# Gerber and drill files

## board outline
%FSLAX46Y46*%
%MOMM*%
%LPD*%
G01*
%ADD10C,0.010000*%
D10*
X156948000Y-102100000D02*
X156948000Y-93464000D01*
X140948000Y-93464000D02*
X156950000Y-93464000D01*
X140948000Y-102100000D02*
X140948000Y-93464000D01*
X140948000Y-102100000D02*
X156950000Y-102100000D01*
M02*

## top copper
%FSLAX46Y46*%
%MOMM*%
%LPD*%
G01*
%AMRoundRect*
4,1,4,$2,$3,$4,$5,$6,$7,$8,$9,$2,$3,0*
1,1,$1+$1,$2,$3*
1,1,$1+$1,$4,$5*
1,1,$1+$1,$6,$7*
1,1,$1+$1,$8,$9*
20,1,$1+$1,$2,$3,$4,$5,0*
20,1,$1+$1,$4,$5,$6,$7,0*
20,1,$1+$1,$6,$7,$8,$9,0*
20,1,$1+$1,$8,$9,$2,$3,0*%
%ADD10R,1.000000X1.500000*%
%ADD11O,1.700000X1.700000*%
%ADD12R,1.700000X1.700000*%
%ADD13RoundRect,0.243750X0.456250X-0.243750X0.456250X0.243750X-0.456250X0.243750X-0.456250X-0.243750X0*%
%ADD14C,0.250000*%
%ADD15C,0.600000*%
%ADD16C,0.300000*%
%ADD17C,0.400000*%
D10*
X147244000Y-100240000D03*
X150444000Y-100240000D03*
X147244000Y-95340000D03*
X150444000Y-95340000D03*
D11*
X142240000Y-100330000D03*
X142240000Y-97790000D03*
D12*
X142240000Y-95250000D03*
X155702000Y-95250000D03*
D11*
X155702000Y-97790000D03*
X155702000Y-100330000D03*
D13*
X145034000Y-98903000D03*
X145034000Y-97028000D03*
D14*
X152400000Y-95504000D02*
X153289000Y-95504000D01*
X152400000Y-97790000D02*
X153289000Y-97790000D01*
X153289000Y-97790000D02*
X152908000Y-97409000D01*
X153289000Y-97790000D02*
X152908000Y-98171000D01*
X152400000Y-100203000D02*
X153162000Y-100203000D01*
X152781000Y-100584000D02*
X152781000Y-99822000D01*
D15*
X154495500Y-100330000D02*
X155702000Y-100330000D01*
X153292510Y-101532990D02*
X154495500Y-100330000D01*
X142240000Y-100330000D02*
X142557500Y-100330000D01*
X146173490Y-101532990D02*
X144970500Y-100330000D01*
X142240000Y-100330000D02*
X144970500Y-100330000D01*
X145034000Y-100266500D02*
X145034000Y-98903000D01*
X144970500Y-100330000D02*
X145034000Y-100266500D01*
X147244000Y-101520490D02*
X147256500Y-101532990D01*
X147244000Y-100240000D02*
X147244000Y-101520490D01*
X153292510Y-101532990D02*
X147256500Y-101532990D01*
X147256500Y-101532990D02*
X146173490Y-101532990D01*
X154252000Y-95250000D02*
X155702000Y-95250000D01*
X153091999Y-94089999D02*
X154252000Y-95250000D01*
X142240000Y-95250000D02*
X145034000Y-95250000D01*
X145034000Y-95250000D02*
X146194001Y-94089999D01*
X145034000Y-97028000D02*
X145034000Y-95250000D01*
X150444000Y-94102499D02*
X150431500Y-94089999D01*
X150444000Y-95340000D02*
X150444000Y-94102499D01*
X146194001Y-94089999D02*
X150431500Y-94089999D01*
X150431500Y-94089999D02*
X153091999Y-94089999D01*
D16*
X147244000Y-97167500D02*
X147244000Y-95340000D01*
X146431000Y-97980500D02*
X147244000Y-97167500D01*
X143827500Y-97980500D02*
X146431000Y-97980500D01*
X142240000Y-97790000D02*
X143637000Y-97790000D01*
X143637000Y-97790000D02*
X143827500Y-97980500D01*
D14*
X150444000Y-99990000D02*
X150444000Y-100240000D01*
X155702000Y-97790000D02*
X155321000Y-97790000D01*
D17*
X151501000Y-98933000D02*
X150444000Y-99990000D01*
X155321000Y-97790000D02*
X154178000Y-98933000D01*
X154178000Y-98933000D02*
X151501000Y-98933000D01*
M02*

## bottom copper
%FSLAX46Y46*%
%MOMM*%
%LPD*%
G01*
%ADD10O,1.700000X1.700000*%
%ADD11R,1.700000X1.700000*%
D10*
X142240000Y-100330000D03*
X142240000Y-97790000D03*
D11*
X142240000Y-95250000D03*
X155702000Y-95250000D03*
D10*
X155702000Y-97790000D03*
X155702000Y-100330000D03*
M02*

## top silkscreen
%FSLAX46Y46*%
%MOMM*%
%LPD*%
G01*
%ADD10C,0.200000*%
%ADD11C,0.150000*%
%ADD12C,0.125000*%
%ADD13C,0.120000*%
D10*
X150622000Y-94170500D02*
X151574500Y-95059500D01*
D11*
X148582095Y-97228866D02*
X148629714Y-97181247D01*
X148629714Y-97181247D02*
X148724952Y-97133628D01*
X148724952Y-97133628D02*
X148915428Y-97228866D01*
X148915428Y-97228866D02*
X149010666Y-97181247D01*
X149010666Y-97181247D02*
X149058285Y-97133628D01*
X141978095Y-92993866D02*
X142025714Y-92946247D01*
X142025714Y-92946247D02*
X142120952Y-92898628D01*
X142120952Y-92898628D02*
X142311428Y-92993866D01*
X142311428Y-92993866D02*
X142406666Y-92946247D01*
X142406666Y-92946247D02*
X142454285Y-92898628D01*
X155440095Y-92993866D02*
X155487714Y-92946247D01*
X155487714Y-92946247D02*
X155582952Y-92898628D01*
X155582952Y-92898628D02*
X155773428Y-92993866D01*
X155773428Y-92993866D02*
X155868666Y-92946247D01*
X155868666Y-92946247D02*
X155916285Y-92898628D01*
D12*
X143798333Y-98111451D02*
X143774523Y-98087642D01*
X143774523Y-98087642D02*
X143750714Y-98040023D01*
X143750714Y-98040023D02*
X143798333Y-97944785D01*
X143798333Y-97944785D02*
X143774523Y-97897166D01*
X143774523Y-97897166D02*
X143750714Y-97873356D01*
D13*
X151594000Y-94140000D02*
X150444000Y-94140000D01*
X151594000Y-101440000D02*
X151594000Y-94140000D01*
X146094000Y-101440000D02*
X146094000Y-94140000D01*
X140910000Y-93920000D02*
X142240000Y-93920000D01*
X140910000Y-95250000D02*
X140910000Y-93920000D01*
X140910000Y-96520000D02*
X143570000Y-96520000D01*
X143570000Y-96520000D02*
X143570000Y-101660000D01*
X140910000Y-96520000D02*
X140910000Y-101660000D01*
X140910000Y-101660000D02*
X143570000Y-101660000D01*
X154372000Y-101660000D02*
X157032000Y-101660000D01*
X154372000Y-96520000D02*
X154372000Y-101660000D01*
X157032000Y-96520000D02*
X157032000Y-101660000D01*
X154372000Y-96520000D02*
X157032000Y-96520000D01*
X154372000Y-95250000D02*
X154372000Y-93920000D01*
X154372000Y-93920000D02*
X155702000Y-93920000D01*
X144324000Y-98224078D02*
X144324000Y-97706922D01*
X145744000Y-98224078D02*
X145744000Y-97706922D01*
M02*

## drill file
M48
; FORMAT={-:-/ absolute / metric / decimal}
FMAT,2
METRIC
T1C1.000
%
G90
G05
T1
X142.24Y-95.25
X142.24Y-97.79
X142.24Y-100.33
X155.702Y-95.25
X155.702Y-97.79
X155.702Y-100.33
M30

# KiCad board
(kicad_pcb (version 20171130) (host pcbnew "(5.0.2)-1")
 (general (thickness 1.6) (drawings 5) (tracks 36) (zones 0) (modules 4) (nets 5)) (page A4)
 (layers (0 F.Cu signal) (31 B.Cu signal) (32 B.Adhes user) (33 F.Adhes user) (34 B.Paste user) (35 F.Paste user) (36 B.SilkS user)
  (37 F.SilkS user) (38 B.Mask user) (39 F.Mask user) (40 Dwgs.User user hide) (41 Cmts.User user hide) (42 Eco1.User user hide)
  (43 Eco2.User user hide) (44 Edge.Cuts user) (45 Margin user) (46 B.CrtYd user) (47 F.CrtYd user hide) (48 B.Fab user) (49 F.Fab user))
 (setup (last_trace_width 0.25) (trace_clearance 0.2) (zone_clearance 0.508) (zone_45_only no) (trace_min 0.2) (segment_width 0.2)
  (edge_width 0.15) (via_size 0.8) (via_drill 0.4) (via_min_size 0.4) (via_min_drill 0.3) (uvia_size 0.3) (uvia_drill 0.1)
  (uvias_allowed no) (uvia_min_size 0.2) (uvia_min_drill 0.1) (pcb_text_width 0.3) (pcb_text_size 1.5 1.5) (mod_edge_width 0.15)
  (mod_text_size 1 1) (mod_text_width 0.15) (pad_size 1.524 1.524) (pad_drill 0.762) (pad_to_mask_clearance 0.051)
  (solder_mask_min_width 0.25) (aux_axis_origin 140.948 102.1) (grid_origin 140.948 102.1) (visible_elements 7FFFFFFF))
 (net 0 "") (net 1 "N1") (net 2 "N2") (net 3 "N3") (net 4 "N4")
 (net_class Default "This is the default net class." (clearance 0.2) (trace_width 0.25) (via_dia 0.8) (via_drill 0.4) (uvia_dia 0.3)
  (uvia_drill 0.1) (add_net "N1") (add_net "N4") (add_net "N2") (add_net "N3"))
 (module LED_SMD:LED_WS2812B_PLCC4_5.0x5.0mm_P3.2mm (layer F.Cu) (at 148.844 97.79 90)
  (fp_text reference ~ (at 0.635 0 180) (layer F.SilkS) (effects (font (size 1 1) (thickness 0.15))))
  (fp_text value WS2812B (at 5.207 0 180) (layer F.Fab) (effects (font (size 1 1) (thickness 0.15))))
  (fp_line (start 3.65 2.75) (end 3.65 1.6) (layer F.SilkS) (width 0.12))
  (fp_line (start -3.65 2.75) (end 3.65 2.75) (layer F.SilkS) (width 0.12))
  (fp_line (start -3.65 -2.75) (end 3.65 -2.75) (layer F.SilkS) (width 0.12))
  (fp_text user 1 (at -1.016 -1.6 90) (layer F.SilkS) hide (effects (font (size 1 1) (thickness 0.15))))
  (pad 1 smd rect (at -2.45 -1.6 90) (size 1.5 1) (layers F.Cu F.Paste F.Mask) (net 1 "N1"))
  (pad 2 smd rect (at -2.45 1.6 90) (size 1.5 1) (layers F.Cu F.Paste F.Mask) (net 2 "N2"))
  (pad 4 smd rect (at 2.45 -1.6 90) (size 1.5 1) (layers F.Cu F.Paste F.Mask) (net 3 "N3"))
  (pad 3 smd rect (at 2.45 1.6 90) (size 1.5 1) (layers F.Cu F.Paste F.Mask) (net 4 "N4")))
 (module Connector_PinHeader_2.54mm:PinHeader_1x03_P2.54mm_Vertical (layer F.Cu) (at 142.24 95.25)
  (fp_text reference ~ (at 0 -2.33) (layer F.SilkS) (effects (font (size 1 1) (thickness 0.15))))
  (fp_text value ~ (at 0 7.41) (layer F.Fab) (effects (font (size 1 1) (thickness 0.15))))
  (fp_line (start -1.33 -1.33) (end 0 -1.33) (layer F.SilkS) (width 0.12))
  (fp_line (start -1.33 0) (end -1.33 -1.33) (layer F.SilkS) (width 0.12))
  (fp_line (start -1.33 1.27) (end 1.33 1.27) (layer F.SilkS) (width 0.12))
  (fp_line (start 1.33 1.27) (end 1.33 6.41) (layer F.SilkS) (width 0.12))
  (fp_line (start -1.33 1.27) (end -1.33 6.41) (layer F.SilkS) (width 0.12))
  (fp_line (start -1.33 6.41) (end 1.33 6.41) (layer F.SilkS) (width 0.12))
  (pad 3 thru_hole oval (at 0 5.08) (size 1.7 1.7) (drill 1) (layers *.Cu *.Mask) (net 1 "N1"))
  (pad 2 thru_hole oval (at 0 2.54) (size 1.7 1.7) (drill 1) (layers *.Cu *.Mask) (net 3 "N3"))
  (pad 1 thru_hole rect (at 0 0) (size 1.7 1.7) (drill 1) (layers *.Cu *.Mask) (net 4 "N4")))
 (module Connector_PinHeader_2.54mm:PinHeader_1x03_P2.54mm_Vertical (layer F.Cu) (at 155.702 95.25)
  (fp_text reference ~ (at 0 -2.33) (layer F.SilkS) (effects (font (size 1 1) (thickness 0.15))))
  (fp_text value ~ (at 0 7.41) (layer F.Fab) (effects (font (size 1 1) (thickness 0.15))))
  (fp_line (start -1.33 6.41) (end 1.33 6.41) (layer F.SilkS) (width 0.12))
  (fp_line (start -1.33 1.27) (end -1.33 6.41) (layer F.SilkS) (width 0.12))
  (fp_line (start 1.33 1.27) (end 1.33 6.41) (layer F.SilkS) (width 0.12))
  (fp_line (start -1.33 1.27) (end 1.33 1.27) (layer F.SilkS) (width 0.12))
  (fp_line (start -1.33 0) (end -1.33 -1.33) (layer F.SilkS) (width 0.12))
  (fp_line (start -1.33 -1.33) (end 0 -1.33) (layer F.SilkS) (width 0.12))
  (pad 1 thru_hole rect (at 0 0) (size 1.7 1.7) (drill 1) (layers *.Cu *.Mask) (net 4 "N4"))
  (pad 2 thru_hole oval (at 0 2.54) (size 1.7 1.7) (drill 1) (layers *.Cu *.Mask) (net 2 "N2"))
  (pad 3 thru_hole oval (at 0 5.08) (size 1.7 1.7) (drill 1) (layers *.Cu *.Mask) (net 1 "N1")))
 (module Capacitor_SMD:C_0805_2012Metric (layer F.Cu) (at 145.034 97.9655 90)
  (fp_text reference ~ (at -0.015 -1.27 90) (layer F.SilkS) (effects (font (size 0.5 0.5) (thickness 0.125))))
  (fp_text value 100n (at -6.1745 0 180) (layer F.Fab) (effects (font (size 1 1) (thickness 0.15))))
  (fp_line (start -0.258578 -0.71) (end 0.258578 -0.71) (layer F.SilkS) (width 0.12))
  (fp_line (start -0.258578 0.71) (end 0.258578 0.71) (layer F.SilkS) (width 0.12))
  (pad 1 smd roundrect (at -0.9375 0 90) (size 0.975 1.4) (layers F.Cu F.Paste F.Mask) (roundrect_rratio 0.25) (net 1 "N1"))
  (pad 2 smd roundrect (at 0.9375 0 90) (size 0.975 1.4) (layers F.Cu F.Paste F.Mask) (roundrect_rratio 0.25) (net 4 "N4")))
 (gr_line (start 156.948 102.1) (end 156.948 93.464) (layer Edge.Cuts) (width 0.01))
 (gr_line (start 150.622 94.1705) (end 151.5745 95.0595) (layer F.SilkS) (width 0.2))
 (gr_line (start 140.948 93.464) (end 156.95 93.464) (layer Edge.Cuts) (width 0.01))
 (gr_line (start 140.948 102.1) (end 140.948 93.464) (layer Edge.Cuts) (width 0.01))
 (gr_line (start 140.948 102.1) (end 156.95 102.1) (layer Edge.Cuts) (width 0.01))
 (segment (start 152.4 95.504) (end 153.289 95.504) (width 0.25) (layer F.Cu) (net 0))
 (segment (start 152.4 97.79) (end 153.289 97.79) (width 0.25) (layer F.Cu) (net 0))
 (segment (start 153.289 97.79) (end 152.908 97.409) (width 0.25) (layer F.Cu) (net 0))
 (segment (start 153.289 97.79) (end 152.908 98.171) (width 0.25) (layer F.Cu) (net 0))
 (segment (start 152.4 100.203) (end 153.162 100.203) (width 0.25) (layer F.Cu) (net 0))
 (segment (start 152.781 100.584) (end 152.781 99.822) (width 0.25) (layer F.Cu) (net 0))
 (segment (start 154.4955 100.33) (end 155.702 100.33) (width 0.6) (layer F.Cu) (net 1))
 (segment (start 153.29251 101.53299) (end 154.4955 100.33) (width 0.6) (layer F.Cu) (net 1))
 (segment (start 142.24 100.33) (end 142.5575 100.33) (width 0.6) (layer F.Cu) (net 1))
 (segment (start 146.17349 101.53299) (end 144.9705 100.33) (width 0.6) (layer F.Cu) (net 1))
 (segment (start 142.24 100.33) (end 144.9705 100.33) (width 0.6) (layer F.Cu) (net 1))
 (segment (start 145.034 100.2665) (end 145.034 98.903) (width 0.6) (layer F.Cu) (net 1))
 (segment (start 144.9705 100.33) (end 145.034 100.2665) (width 0.6) (layer F.Cu) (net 1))
 (segment (start 147.244 101.52049) (end 147.2565 101.53299) (width 0.6) (layer F.Cu) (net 1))
 (segment (start 147.244 100.24) (end 147.244 101.52049) (width 0.6) (layer F.Cu) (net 1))
 (segment (start 153.29251 101.53299) (end 147.2565 101.53299) (width 0.6) (layer F.Cu) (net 1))
 (segment (start 147.2565 101.53299) (end 146.17349 101.53299) (width 0.6) (layer F.Cu) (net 1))
 (segment (start 154.252 95.25) (end 155.702 95.25) (width 0.6) (layer F.Cu) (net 4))
 (segment (start 153.091999 94.089999) (end 154.252 95.25) (width 0.6) (layer F.Cu) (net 4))
 (segment (start 142.24 95.25) (end 145.034 95.25) (width 0.6) (layer F.Cu) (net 4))
 (segment (start 145.034 95.25) (end 146.194001 94.089999) (width 0.6) (layer F.Cu) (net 4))
 (segment (start 145.034 97.028) (end 145.034 95.25) (width 0.6) (layer F.Cu) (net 4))
 (segment (start 150.444 94.102499) (end 150.4315 94.089999) (width 0.6) (layer F.Cu) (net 4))
 (segment (start 150.444 95.34) (end 150.444 94.102499) (width 0.6) (layer F.Cu) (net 4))
 (segment (start 146.194001 94.089999) (end 150.4315 94.089999) (width 0.6) (layer F.Cu) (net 4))
 (segment (start 150.4315 94.089999) (end 153.091999 94.089999) (width 0.6) (layer F.Cu) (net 4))
 (segment (start 147.244 97.1675) (end 147.244 95.34) (width 0.3) (layer F.Cu) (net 3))
 (segment (start 146.431 97.9805) (end 147.244 97.1675) (width 0.3) (layer F.Cu) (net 3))
 (segment (start 143.8275 97.9805) (end 146.431 97.9805) (width 0.3) (layer F.Cu) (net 3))
 (segment (start 142.24 97.79) (end 143.637 97.79) (width 0.3) (layer F.Cu) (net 3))
 (segment (start 143.637 97.79) (end 143.8275 97.9805) (width 0.3) (layer F.Cu) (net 3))
 (segment (start 150.444 99.99) (end 150.444 100.24) (width 0.25) (layer F.Cu) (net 2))
 (segment (start 155.702 97.79) (end 155.321 97.79) (width 0.25) (layer F.Cu) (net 2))
 (segment (start 151.501 98.933) (end 150.444 99.99) (width 0.4) (layer F.Cu) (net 2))
 (segment (start 155.321 97.79) (end 154.178 98.933) (width 0.4) (layer F.Cu) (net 2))
 (segment (start 154.178 98.933) (end 151.501 98.933) (width 0.4) (layer F.Cu) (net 2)))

